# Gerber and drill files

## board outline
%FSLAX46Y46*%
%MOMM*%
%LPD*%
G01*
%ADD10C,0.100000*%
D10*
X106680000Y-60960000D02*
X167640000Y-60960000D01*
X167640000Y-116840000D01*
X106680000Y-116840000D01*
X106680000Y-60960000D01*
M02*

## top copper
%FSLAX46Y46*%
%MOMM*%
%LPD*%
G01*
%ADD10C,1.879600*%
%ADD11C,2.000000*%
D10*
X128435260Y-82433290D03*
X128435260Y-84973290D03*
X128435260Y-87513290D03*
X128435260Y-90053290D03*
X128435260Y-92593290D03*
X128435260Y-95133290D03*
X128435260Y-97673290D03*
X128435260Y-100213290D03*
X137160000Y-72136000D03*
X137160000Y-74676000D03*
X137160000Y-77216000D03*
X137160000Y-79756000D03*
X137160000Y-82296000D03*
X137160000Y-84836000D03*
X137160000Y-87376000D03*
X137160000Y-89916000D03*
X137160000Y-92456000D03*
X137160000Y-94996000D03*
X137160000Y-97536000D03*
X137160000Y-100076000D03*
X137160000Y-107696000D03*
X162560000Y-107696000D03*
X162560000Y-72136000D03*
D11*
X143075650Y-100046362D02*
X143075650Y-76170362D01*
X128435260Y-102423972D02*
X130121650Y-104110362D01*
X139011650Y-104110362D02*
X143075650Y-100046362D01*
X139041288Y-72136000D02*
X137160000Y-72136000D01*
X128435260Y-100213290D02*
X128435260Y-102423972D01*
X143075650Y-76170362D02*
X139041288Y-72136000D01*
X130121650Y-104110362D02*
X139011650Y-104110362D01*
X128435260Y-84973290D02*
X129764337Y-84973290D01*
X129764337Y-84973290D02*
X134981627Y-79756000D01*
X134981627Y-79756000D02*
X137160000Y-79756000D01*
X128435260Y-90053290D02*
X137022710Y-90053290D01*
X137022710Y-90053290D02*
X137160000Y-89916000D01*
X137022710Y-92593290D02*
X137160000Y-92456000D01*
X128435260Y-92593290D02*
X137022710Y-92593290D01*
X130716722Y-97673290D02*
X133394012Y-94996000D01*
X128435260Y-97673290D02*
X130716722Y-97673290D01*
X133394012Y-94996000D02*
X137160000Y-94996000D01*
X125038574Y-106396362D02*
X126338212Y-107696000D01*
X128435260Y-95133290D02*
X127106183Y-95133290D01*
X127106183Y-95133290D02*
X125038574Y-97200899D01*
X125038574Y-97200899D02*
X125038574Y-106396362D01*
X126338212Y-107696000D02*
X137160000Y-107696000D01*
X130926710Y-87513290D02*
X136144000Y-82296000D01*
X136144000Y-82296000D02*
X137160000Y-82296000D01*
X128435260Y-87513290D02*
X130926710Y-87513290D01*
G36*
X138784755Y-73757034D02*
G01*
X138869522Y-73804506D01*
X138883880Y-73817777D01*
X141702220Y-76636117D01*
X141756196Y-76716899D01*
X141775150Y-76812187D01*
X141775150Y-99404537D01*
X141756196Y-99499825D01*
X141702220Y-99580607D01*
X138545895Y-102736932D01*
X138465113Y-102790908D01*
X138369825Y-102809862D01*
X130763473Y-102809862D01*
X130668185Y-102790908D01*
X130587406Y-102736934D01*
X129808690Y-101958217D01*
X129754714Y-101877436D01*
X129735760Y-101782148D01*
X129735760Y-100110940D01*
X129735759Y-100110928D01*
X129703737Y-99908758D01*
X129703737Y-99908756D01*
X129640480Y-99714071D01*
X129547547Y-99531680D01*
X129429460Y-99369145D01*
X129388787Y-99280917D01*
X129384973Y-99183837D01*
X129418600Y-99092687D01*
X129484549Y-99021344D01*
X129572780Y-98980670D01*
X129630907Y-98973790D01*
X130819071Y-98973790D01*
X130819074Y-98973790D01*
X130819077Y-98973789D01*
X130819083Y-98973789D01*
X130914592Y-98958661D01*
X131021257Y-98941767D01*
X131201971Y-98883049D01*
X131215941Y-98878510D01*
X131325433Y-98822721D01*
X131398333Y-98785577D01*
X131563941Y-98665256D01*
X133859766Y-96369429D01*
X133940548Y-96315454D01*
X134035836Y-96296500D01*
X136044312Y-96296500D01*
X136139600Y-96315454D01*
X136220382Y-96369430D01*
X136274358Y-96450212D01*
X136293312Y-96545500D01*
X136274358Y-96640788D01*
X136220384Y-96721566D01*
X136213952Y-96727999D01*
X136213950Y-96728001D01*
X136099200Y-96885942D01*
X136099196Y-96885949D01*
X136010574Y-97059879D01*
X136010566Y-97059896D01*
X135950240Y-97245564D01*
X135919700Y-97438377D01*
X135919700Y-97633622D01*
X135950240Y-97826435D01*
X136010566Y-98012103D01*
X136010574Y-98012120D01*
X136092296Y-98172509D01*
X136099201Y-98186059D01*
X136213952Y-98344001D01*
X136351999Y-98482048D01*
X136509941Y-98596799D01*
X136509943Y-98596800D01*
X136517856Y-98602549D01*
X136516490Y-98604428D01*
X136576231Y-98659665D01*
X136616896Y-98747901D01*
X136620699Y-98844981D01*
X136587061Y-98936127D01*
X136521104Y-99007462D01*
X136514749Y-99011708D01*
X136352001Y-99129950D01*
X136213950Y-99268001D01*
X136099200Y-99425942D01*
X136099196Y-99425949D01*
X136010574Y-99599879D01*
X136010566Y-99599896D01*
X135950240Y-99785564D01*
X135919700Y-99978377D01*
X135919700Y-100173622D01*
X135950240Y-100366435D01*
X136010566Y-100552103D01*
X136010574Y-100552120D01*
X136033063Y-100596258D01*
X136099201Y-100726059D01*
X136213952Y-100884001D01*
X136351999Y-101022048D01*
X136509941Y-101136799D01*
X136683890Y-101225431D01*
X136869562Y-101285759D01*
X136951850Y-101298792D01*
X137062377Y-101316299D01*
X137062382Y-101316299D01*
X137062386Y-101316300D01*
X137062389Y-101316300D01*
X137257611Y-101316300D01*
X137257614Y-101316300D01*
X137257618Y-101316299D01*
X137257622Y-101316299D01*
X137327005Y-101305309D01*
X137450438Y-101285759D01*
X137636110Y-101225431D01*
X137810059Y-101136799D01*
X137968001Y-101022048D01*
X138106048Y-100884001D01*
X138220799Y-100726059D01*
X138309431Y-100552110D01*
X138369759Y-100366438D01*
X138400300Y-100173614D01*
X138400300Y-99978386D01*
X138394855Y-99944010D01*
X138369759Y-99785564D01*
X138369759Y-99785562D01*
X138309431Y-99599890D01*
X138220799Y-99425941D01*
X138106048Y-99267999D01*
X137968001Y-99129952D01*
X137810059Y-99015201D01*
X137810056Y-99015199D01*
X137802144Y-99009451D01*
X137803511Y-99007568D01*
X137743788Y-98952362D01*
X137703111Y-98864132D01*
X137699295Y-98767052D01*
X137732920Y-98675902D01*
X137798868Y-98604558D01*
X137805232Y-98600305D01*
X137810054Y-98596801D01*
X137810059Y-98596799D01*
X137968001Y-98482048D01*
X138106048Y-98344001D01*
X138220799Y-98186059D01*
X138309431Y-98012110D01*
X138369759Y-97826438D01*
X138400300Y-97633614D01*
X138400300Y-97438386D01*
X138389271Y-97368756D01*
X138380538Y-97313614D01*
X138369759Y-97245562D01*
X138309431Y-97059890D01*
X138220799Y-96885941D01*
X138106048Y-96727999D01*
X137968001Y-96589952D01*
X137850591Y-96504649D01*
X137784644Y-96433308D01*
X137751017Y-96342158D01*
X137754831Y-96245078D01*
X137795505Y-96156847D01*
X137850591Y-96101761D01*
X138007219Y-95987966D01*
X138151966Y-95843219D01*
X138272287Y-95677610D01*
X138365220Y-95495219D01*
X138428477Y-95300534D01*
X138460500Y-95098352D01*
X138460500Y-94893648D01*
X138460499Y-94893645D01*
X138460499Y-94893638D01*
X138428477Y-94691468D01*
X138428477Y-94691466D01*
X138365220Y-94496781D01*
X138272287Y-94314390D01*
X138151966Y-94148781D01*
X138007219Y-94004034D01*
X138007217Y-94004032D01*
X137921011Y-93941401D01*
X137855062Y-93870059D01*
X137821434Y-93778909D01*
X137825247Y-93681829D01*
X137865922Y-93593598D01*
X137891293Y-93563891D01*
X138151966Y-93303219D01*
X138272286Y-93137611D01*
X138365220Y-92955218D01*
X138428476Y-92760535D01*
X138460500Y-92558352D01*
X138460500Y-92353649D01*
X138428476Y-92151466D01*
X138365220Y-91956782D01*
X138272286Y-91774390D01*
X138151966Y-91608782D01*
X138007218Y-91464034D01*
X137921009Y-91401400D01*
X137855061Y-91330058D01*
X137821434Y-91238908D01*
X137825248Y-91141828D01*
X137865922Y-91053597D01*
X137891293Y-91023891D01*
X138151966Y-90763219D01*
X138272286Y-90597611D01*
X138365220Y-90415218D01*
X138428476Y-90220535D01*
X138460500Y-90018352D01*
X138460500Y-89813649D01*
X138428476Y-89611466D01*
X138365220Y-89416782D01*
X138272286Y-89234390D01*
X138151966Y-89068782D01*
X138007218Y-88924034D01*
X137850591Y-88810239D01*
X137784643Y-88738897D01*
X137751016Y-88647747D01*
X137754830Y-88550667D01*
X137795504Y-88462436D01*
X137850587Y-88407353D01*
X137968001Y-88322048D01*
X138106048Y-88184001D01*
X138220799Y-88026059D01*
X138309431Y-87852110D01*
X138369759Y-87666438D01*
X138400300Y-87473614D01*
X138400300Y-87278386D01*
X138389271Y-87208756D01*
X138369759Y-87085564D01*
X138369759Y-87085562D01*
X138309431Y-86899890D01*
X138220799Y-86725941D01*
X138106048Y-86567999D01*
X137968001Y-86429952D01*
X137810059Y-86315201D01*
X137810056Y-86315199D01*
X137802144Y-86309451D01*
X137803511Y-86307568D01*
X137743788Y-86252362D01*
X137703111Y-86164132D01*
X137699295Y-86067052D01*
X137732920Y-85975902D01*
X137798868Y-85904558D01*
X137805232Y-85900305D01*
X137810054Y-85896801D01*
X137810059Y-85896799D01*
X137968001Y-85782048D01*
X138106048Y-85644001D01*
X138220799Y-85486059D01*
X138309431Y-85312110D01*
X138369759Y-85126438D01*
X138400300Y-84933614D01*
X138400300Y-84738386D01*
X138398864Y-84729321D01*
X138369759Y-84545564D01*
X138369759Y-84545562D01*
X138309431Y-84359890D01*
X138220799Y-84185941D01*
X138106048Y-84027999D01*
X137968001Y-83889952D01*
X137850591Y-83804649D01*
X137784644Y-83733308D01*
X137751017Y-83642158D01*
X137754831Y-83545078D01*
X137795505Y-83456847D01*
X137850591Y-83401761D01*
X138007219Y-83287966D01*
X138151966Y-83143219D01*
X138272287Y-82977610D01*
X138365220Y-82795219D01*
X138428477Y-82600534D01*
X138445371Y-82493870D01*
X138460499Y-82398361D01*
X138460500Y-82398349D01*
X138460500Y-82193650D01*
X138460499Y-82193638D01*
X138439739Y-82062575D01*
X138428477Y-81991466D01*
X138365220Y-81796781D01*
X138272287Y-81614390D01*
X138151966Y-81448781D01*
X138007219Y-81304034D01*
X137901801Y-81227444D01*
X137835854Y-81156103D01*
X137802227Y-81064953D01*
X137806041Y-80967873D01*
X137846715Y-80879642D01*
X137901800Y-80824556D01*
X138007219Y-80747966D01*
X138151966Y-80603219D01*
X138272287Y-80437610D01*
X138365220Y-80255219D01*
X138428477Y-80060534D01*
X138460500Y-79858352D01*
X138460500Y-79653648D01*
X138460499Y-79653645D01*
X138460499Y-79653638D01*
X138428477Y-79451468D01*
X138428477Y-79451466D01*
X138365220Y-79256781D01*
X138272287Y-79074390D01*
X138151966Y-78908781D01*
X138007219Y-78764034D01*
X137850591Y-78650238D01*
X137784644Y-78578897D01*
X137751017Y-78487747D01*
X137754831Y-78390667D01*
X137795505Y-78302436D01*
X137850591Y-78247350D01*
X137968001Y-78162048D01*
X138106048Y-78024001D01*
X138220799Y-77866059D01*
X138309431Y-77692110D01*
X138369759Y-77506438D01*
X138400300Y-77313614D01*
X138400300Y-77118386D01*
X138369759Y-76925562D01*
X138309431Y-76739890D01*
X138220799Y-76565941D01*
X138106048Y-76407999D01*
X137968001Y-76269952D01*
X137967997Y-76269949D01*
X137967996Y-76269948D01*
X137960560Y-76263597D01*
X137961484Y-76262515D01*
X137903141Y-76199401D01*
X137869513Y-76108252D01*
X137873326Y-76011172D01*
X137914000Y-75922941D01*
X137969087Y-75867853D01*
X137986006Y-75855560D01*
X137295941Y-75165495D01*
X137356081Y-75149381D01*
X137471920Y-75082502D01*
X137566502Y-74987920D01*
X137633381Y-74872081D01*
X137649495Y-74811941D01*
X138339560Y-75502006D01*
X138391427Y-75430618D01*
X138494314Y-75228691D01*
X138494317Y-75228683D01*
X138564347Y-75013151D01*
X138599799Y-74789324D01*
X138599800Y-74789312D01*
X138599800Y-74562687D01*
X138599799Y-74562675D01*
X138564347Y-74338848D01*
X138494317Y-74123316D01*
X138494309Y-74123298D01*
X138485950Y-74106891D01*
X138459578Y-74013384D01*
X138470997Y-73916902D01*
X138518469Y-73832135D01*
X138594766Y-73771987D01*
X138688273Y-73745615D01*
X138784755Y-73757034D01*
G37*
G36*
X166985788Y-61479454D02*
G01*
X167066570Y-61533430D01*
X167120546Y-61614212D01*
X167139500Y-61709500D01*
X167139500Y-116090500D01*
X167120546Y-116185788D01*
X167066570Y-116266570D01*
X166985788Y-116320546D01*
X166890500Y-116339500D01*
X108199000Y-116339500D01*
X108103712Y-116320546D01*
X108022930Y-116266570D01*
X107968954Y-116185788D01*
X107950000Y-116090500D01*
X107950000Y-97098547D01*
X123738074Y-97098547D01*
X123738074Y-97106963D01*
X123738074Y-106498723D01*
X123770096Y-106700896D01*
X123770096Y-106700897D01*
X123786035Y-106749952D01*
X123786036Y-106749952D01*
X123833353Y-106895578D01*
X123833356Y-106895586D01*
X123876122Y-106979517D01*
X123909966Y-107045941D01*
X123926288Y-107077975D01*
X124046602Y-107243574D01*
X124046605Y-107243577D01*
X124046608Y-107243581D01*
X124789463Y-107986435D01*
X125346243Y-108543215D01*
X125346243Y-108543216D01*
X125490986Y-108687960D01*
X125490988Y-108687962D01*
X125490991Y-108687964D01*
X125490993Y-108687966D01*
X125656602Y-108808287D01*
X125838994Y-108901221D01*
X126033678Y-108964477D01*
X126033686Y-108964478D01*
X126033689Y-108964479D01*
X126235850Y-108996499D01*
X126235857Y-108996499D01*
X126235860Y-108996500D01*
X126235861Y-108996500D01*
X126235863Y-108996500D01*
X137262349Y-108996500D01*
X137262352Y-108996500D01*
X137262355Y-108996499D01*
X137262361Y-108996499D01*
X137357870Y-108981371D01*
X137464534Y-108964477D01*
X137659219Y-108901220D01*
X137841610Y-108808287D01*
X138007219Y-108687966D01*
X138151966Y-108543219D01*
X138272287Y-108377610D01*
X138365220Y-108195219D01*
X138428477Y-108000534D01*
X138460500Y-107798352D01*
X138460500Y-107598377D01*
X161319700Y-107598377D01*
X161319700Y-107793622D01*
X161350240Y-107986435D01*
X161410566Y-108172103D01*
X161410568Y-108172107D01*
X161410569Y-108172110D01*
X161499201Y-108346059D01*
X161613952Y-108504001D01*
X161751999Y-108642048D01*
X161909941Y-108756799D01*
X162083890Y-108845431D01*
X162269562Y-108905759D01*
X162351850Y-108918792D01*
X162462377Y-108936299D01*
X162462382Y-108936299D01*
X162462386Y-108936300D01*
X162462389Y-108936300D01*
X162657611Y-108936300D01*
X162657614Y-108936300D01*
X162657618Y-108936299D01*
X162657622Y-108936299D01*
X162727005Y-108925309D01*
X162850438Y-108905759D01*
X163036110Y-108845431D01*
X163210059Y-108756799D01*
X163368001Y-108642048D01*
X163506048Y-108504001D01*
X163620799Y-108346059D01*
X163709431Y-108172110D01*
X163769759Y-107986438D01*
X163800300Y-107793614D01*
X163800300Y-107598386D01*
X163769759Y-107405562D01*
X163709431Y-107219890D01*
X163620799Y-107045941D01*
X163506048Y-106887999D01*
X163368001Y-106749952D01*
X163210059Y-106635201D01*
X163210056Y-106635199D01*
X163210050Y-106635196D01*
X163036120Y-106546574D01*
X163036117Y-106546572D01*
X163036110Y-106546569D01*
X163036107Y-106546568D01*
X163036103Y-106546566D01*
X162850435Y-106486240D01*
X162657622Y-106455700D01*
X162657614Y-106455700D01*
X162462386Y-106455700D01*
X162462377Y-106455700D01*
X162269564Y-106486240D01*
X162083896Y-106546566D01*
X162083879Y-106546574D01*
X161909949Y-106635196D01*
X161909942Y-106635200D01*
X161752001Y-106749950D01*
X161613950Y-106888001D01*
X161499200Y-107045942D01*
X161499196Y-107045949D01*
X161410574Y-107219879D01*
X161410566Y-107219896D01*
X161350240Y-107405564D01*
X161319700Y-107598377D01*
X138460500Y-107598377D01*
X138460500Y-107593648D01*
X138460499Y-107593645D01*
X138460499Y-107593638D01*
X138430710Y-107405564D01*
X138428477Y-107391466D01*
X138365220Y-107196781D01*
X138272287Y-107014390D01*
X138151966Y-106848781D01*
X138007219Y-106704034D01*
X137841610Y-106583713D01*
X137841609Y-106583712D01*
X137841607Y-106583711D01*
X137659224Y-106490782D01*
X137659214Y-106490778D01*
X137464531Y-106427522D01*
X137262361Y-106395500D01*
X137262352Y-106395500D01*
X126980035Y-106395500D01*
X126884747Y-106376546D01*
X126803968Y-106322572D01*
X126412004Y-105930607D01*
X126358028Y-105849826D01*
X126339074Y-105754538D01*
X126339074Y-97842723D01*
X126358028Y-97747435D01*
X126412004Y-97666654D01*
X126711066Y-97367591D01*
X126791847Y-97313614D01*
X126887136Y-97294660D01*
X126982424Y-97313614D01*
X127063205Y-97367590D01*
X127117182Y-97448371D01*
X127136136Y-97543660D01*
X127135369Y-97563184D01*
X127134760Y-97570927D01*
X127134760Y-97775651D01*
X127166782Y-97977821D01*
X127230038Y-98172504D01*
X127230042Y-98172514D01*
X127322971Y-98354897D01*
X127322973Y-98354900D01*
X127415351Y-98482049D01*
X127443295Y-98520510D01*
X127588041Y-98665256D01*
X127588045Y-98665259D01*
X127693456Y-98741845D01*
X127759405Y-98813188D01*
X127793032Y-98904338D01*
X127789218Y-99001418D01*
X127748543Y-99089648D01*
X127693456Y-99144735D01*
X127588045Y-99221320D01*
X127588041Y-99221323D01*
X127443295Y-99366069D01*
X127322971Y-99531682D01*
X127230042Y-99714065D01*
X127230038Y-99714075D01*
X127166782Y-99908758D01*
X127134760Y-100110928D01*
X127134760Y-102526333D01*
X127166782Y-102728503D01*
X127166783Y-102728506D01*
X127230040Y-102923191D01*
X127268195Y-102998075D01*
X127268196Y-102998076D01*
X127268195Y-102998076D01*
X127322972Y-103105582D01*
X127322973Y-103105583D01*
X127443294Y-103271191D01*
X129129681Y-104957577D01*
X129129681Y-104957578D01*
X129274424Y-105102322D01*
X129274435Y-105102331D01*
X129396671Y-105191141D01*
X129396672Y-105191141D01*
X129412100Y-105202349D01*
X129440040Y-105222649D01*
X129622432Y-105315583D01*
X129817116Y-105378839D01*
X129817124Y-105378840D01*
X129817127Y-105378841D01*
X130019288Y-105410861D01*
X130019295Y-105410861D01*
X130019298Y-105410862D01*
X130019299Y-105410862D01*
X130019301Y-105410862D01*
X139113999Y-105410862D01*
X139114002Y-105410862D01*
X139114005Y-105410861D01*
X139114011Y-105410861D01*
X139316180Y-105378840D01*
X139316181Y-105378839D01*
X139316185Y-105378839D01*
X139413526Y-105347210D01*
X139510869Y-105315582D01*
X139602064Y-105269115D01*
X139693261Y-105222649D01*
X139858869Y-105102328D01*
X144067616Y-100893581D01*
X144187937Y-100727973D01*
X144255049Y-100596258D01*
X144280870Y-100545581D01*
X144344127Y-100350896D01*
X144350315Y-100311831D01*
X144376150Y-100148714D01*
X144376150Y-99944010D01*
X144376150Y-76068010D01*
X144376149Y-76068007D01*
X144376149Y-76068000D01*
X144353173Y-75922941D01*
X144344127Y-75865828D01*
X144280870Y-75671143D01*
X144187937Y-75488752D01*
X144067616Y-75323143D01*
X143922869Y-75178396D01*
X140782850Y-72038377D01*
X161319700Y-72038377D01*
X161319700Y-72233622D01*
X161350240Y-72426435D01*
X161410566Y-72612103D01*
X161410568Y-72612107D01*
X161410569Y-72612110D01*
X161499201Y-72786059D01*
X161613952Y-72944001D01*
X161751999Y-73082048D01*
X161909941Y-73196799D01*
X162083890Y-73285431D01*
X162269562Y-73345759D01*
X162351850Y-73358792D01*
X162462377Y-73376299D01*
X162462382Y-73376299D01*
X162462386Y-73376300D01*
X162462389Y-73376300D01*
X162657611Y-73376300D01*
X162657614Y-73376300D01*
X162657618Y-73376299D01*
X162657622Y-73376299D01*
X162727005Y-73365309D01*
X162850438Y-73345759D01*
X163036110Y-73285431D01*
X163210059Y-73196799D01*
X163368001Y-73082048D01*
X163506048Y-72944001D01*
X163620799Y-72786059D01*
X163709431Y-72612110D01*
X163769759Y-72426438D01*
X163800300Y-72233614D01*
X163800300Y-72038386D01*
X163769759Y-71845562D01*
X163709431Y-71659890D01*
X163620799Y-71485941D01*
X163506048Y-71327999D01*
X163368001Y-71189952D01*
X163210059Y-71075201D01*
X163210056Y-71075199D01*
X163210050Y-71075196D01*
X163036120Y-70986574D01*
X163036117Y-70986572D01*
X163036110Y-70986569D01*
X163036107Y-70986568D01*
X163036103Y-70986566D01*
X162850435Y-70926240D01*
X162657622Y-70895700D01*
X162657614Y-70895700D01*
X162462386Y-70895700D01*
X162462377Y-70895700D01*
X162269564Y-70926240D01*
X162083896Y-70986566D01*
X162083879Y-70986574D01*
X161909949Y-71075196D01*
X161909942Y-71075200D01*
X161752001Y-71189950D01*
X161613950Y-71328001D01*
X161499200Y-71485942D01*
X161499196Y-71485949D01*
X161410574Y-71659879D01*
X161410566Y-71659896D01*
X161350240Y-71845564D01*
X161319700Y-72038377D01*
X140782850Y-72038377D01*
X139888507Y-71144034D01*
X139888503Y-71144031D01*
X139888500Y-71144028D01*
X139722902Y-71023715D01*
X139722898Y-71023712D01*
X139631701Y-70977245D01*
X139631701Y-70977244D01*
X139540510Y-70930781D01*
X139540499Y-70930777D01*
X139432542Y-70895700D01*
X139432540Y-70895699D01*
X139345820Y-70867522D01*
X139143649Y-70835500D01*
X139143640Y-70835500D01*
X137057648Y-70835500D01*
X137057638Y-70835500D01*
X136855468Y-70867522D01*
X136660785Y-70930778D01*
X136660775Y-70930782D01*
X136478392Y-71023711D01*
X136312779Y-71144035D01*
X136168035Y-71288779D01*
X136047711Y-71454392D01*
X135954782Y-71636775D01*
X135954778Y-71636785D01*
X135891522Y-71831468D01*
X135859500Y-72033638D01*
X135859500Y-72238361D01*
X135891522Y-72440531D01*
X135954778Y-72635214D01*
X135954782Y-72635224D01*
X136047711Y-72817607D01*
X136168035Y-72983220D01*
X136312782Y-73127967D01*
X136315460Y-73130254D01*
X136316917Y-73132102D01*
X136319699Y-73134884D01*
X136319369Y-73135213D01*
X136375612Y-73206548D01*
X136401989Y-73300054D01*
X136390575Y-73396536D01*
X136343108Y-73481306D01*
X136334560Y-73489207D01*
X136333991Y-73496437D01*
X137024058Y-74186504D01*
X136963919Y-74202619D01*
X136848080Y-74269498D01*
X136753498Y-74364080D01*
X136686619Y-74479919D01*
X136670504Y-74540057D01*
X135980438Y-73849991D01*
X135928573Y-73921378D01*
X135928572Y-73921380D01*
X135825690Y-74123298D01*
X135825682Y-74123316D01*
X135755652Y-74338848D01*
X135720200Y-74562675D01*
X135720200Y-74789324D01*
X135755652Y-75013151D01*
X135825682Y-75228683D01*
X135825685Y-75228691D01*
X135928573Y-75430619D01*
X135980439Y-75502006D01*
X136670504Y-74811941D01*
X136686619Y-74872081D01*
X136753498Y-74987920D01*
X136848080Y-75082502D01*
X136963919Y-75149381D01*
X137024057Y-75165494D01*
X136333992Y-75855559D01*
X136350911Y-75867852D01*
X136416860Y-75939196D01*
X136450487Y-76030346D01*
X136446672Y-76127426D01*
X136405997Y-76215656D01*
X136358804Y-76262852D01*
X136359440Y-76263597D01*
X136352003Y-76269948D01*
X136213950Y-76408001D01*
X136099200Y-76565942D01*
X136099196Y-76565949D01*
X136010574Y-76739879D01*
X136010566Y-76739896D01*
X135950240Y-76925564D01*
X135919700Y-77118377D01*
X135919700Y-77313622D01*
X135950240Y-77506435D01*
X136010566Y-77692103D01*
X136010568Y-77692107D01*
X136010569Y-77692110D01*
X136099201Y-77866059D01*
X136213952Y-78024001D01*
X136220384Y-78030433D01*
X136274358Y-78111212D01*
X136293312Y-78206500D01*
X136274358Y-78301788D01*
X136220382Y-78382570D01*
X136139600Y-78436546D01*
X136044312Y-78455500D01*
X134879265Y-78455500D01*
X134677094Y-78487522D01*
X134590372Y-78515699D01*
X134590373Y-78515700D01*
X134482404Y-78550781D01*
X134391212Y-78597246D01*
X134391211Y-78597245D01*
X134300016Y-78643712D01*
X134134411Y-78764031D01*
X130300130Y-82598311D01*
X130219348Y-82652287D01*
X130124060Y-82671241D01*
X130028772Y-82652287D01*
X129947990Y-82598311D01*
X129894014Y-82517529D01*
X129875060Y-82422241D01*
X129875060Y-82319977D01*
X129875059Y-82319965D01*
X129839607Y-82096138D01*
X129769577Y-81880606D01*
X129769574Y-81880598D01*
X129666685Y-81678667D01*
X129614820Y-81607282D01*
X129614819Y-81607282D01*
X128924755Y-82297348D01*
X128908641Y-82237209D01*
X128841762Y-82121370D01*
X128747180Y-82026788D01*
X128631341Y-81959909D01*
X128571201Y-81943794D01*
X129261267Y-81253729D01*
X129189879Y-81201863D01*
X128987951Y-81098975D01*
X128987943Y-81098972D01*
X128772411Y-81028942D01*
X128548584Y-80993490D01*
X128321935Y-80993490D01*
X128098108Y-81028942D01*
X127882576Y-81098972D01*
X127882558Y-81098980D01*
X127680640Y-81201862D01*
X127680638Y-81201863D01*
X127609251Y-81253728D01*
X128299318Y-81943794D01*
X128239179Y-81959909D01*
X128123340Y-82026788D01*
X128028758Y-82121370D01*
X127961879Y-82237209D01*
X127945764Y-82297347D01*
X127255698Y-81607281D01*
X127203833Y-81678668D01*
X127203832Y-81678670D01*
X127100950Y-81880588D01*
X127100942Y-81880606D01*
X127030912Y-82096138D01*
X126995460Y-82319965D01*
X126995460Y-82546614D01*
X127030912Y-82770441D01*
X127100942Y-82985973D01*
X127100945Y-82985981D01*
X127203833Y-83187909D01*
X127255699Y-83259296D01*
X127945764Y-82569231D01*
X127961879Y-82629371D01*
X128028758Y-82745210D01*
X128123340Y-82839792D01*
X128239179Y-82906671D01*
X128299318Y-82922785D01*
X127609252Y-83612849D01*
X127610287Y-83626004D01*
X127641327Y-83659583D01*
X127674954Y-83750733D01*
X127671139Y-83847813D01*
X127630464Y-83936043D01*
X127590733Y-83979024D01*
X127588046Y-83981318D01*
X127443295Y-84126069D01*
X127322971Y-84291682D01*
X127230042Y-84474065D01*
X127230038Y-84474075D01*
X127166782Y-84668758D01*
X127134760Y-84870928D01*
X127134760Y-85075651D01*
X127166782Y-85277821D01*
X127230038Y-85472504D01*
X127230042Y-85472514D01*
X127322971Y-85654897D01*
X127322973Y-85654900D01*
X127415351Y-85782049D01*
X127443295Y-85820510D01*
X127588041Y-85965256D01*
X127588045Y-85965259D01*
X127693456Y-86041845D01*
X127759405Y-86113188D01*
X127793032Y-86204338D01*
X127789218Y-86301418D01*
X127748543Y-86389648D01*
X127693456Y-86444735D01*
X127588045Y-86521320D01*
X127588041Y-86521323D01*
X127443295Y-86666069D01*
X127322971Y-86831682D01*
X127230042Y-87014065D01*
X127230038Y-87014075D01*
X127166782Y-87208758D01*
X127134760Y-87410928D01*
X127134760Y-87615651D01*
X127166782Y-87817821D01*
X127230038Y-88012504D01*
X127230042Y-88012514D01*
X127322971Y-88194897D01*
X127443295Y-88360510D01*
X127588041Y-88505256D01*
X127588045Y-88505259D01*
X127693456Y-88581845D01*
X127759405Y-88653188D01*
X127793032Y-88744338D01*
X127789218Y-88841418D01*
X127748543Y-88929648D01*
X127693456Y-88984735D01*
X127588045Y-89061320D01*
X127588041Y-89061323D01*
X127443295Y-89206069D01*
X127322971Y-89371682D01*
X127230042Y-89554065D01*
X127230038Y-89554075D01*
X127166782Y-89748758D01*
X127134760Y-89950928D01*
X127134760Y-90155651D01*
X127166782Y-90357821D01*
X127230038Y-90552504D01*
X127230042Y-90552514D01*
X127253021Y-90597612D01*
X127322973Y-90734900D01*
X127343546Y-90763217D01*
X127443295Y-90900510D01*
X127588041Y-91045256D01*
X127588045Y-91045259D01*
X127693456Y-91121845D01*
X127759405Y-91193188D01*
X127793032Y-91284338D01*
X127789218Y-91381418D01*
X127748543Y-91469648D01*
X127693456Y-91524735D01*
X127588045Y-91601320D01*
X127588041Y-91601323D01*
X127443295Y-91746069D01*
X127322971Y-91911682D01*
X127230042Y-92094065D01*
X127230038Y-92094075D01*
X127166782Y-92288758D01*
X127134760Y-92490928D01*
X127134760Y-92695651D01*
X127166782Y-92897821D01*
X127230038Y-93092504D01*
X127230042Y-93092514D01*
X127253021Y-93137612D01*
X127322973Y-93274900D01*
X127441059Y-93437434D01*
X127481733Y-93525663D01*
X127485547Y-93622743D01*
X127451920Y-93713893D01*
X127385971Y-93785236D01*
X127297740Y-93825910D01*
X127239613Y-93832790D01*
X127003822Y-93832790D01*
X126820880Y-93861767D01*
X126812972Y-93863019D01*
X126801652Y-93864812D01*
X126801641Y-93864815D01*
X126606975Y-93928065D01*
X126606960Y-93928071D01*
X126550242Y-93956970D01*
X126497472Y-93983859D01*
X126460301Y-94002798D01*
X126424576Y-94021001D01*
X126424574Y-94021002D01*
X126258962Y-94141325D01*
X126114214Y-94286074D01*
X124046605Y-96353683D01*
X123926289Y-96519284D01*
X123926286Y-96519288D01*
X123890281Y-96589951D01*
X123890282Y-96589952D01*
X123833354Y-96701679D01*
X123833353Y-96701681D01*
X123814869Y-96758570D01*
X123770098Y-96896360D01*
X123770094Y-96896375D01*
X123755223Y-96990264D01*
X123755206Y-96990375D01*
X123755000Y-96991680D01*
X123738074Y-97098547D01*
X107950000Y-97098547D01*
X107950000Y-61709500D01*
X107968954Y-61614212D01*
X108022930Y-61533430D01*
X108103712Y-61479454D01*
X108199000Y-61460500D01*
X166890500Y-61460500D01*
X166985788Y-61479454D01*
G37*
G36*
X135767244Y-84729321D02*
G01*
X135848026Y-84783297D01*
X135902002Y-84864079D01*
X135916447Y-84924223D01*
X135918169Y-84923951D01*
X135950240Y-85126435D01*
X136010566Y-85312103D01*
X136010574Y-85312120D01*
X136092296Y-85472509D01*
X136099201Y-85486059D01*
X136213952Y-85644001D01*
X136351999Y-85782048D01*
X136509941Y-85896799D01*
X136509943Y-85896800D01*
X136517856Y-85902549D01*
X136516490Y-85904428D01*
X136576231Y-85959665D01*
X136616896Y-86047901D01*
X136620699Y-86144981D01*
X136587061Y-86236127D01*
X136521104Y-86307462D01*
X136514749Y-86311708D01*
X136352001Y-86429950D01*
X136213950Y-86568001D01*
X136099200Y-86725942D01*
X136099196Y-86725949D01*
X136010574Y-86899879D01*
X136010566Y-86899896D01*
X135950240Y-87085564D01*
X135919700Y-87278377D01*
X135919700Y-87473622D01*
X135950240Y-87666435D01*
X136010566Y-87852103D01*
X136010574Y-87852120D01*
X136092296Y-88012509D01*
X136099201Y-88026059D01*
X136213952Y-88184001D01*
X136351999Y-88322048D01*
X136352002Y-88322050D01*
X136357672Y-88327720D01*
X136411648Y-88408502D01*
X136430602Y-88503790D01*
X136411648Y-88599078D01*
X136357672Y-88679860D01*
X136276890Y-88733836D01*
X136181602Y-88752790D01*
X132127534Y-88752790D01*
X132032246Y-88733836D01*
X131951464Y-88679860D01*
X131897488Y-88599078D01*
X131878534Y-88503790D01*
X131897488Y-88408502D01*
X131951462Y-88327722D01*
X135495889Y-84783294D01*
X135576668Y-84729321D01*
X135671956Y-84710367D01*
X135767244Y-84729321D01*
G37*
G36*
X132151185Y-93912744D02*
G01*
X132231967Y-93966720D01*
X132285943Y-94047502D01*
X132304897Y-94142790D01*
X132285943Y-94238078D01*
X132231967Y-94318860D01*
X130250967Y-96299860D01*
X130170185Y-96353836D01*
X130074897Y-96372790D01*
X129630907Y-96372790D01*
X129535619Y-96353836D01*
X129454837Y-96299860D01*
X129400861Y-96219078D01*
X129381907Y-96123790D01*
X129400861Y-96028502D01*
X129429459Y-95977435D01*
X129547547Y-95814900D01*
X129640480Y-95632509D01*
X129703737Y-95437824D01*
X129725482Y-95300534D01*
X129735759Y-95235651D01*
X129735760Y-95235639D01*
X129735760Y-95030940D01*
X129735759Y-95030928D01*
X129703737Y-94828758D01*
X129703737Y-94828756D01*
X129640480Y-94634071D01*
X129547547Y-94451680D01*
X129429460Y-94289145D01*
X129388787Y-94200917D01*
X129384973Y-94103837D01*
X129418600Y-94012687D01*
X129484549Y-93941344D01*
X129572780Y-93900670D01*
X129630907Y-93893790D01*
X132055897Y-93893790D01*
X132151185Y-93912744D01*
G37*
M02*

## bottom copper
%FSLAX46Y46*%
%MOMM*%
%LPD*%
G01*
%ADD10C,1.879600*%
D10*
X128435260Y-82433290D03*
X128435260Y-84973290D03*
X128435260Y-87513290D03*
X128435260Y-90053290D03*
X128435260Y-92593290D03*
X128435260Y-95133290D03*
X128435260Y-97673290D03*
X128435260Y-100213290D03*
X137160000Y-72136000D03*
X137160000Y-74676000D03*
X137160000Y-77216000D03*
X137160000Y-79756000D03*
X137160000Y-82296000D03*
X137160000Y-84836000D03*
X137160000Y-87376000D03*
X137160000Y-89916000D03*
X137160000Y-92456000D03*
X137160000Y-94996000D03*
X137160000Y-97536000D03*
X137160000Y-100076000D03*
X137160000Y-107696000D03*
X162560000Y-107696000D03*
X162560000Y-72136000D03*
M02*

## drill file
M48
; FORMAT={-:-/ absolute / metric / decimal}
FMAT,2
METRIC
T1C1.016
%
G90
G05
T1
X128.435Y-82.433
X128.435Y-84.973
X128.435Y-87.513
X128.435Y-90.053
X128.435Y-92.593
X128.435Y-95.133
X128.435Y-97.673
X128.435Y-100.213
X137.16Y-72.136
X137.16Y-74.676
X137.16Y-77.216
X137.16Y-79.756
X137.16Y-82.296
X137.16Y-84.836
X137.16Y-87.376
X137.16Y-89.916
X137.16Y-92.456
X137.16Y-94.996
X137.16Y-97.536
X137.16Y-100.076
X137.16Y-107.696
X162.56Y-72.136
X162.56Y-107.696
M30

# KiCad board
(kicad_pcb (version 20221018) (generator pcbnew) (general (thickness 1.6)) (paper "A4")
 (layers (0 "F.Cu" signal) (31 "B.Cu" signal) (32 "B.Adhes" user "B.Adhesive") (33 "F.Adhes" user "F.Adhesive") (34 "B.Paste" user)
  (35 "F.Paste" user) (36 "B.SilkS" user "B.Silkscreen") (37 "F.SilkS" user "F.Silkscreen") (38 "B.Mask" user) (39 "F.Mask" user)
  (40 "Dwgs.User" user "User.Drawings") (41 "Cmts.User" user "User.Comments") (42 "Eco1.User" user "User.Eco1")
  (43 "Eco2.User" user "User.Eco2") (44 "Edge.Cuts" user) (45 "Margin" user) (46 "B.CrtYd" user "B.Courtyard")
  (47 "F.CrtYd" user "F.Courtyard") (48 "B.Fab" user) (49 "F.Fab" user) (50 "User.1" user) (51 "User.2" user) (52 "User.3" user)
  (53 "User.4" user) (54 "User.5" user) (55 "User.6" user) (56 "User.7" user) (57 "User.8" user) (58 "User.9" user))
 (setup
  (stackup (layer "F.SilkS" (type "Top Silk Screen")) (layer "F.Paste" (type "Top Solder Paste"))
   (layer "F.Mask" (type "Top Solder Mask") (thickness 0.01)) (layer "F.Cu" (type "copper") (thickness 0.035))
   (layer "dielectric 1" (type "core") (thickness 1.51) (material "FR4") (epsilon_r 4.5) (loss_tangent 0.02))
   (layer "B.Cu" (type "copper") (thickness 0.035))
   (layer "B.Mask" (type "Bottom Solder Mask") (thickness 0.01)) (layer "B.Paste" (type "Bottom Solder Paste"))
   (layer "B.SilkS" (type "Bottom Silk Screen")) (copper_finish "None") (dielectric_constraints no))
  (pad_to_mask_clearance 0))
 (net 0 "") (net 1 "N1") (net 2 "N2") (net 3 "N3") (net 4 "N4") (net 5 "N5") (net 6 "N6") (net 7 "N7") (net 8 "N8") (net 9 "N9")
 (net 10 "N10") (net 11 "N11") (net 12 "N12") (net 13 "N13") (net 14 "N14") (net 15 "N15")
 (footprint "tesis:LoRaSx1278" (layer "F.Cu") (at 120.81526 92.59329 -90)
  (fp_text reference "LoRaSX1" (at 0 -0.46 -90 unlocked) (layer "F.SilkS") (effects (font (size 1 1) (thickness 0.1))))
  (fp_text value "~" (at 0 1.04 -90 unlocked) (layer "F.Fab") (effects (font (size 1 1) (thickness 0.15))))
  (pad "1" thru_hole circle (at -10.16 -7.62 270) (size 1.8796 1.8796) (drill 1.016) (layers "*.Cu" "*.Mask") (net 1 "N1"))
  (pad "2" thru_hole circle (at -7.62 -7.62 270) (size 1.8796 1.8796) (drill 1.016) (layers "*.Cu" "*.Mask") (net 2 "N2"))
  (pad "3" thru_hole circle (at -5.08 -7.62 270) (size 1.8796 1.8796) (drill 1.016) (layers "*.Cu" "*.Mask") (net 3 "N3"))
  (pad "4" thru_hole circle (at -2.54 -7.62 270) (size 1.8796 1.8796) (drill 1.016) (layers "*.Cu" "*.Mask") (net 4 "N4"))
  (pad "5" thru_hole circle (at 0 -7.62 270) (size 1.8796 1.8796) (drill 1.016) (layers "*.Cu" "*.Mask") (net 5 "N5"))
  (pad "6" thru_hole circle (at 2.54 -7.62 270) (size 1.8796 1.8796) (drill 1.016) (layers "*.Cu" "*.Mask") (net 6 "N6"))
  (pad "7" thru_hole circle (at 5.08 -7.62 270) (size 1.8796 1.8796) (drill 1.016) (layers "*.Cu" "*.Mask") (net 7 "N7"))
  (pad "8" thru_hole circle (at 7.62 -7.62 270) (size 1.8796 1.8796) (drill 1.016) (layers "*.Cu" "*.Mask") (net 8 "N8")))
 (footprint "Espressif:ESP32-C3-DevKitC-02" (layer "F.Cu") (at 137.16 72.136)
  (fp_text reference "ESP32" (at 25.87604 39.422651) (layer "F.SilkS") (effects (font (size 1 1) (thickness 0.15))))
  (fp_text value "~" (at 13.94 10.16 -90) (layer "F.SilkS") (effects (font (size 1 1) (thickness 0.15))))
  (pad "1" thru_hole circle (at 0 0 270) (size 1.8796 1.8796) (drill 1.016) (layers "*.Cu" "*.Mask") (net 8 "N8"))
  (pad "2" thru_hole circle (at 0 2.54 270) (size 1.8796 1.8796) (drill 1.016) (layers "*.Cu" "*.Mask") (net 1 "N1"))
  (pad "3" thru_hole circle (at 0 5.08 270) (size 1.8796 1.8796) (drill 1.016) (layers "*.Cu" "*.Mask") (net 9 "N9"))
  (pad "4" thru_hole circle (at 0 7.62 270) (size 1.8796 1.8796) (drill 1.016) (layers "*.Cu" "*.Mask") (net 2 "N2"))
  (pad "5" thru_hole circle (at 0 10.16 270) (size 1.8796 1.8796) (drill 1.016) (layers "*.Cu" "*.Mask") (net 3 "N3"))
  (pad "6" thru_hole circle (at 0 12.7 270) (size 1.8796 1.8796) (drill 1.016) (layers "*.Cu" "*.Mask") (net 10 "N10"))
  (pad "7" thru_hole circle (at 0 15.24 270) (size 1.8796 1.8796) (drill 1.016) (layers "*.Cu" "*.Mask") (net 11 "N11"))
  (pad "8" thru_hole circle (at 0 17.78 270) (size 1.8796 1.8796) (drill 1.016) (layers "*.Cu" "*.Mask") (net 4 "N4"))
  (pad "9" thru_hole circle (at 0 20.32 270) (size 1.8796 1.8796) (drill 1.016) (layers "*.Cu" "*.Mask") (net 5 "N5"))
  (pad "10" thru_hole circle (at 0 22.86 270) (size 1.8796 1.8796) (drill 1.016) (layers "*.Cu" "*.Mask") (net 7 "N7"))
  (pad "11" thru_hole circle (at 0 25.4 270) (size 1.8796 1.8796) (drill 1.016) (layers "*.Cu" "*.Mask") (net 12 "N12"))
  (pad "12" thru_hole circle (at 0 27.94 270) (size 1.8796 1.8796) (drill 1.016) (layers "*.Cu" "*.Mask") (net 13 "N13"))
  (pad "15" thru_hole circle (at 0 35.56 270) (size 1.8796 1.8796) (drill 1.016) (layers "*.Cu" "*.Mask") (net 6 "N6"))
  (pad "16" thru_hole circle (at 25.4 35.56 270) (size 1.8796 1.8796) (drill 1.016) (layers "*.Cu" "*.Mask") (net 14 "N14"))
  (pad "30" thru_hole circle (at 25.4 0 270) (size 1.8796 1.8796) (drill 1.016) (layers "*.Cu" "*.Mask") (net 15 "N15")))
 (gr_rect (start 106.68 60.96) (end 167.64 116.84) (stroke (width 0.1) (type default)) (fill none) (layer "Edge.Cuts"))
 (segment (start 143.07565 100.046362) (end 143.07565 76.170362) (width 2) (layer "F.Cu") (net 8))
 (segment (start 128.43526 102.423972) (end 130.12165 104.110362) (width 2) (layer "F.Cu") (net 8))
 (segment (start 139.01165 104.110362) (end 143.07565 100.046362) (width 2) (layer "F.Cu") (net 8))
 (segment (start 139.041288 72.136) (end 137.16 72.136) (width 2) (layer "F.Cu") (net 8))
 (segment (start 128.43526 100.21329) (end 128.43526 102.423972) (width 2) (layer "F.Cu") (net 8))
 (segment (start 143.07565 76.170362) (end 139.041288 72.136) (width 2) (layer "F.Cu") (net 8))
 (segment (start 130.12165 104.110362) (end 139.01165 104.110362) (width 2) (layer "F.Cu") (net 8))
 (segment (start 128.43526 84.97329) (end 129.764337 84.97329) (width 2) (layer "F.Cu") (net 2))
 (segment (start 129.764337 84.97329) (end 134.981627 79.756) (width 2) (layer "F.Cu") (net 2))
 (segment (start 134.981627 79.756) (end 137.16 79.756) (width 2) (layer "F.Cu") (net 2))
 (segment (start 128.43526 90.05329) (end 137.02271 90.05329) (width 2) (layer "F.Cu") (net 4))
 (segment (start 137.02271 90.05329) (end 137.16 89.916) (width 2) (layer "F.Cu") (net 4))
 (segment (start 137.02271 92.59329) (end 137.16 92.456) (width 2) (layer "F.Cu") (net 5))
 (segment (start 128.43526 92.59329) (end 137.02271 92.59329) (width 2) (layer "F.Cu") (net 5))
 (segment (start 130.716722 97.67329) (end 133.394012 94.996) (width 2) (layer "F.Cu") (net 7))
 (segment (start 128.43526 97.67329) (end 130.716722 97.67329) (width 2) (layer "F.Cu") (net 7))
 (segment (start 133.394012 94.996) (end 137.16 94.996) (width 2) (layer "F.Cu") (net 7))
 (segment (start 125.038574 106.396362) (end 126.338212 107.696) (width 2) (layer "F.Cu") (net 6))
 (segment (start 128.43526 95.13329) (end 127.106183 95.13329) (width 2) (layer "F.Cu") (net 6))
 (segment (start 127.106183 95.13329) (end 125.038574 97.200899) (width 2) (layer "F.Cu") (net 6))
 (segment (start 125.038574 97.200899) (end 125.038574 106.396362) (width 2) (layer "F.Cu") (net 6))
 (segment (start 126.338212 107.696) (end 137.16 107.696) (width 2) (layer "F.Cu") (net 6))
 (segment (start 130.92671 87.51329) (end 136.144 82.296) (width 2) (layer "F.Cu") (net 3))
 (segment (start 136.144 82.296) (end 137.16 82.296) (width 2) (layer "F.Cu") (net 3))
 (segment (start 128.43526 87.51329) (end 130.92671 87.51329) (width 2) (layer "F.Cu") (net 3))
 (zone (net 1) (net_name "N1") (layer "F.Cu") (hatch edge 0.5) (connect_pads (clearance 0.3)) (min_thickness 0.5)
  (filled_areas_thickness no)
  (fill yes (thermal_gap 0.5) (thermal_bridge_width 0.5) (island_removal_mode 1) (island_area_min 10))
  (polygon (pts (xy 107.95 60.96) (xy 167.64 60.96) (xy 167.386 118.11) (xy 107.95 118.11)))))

